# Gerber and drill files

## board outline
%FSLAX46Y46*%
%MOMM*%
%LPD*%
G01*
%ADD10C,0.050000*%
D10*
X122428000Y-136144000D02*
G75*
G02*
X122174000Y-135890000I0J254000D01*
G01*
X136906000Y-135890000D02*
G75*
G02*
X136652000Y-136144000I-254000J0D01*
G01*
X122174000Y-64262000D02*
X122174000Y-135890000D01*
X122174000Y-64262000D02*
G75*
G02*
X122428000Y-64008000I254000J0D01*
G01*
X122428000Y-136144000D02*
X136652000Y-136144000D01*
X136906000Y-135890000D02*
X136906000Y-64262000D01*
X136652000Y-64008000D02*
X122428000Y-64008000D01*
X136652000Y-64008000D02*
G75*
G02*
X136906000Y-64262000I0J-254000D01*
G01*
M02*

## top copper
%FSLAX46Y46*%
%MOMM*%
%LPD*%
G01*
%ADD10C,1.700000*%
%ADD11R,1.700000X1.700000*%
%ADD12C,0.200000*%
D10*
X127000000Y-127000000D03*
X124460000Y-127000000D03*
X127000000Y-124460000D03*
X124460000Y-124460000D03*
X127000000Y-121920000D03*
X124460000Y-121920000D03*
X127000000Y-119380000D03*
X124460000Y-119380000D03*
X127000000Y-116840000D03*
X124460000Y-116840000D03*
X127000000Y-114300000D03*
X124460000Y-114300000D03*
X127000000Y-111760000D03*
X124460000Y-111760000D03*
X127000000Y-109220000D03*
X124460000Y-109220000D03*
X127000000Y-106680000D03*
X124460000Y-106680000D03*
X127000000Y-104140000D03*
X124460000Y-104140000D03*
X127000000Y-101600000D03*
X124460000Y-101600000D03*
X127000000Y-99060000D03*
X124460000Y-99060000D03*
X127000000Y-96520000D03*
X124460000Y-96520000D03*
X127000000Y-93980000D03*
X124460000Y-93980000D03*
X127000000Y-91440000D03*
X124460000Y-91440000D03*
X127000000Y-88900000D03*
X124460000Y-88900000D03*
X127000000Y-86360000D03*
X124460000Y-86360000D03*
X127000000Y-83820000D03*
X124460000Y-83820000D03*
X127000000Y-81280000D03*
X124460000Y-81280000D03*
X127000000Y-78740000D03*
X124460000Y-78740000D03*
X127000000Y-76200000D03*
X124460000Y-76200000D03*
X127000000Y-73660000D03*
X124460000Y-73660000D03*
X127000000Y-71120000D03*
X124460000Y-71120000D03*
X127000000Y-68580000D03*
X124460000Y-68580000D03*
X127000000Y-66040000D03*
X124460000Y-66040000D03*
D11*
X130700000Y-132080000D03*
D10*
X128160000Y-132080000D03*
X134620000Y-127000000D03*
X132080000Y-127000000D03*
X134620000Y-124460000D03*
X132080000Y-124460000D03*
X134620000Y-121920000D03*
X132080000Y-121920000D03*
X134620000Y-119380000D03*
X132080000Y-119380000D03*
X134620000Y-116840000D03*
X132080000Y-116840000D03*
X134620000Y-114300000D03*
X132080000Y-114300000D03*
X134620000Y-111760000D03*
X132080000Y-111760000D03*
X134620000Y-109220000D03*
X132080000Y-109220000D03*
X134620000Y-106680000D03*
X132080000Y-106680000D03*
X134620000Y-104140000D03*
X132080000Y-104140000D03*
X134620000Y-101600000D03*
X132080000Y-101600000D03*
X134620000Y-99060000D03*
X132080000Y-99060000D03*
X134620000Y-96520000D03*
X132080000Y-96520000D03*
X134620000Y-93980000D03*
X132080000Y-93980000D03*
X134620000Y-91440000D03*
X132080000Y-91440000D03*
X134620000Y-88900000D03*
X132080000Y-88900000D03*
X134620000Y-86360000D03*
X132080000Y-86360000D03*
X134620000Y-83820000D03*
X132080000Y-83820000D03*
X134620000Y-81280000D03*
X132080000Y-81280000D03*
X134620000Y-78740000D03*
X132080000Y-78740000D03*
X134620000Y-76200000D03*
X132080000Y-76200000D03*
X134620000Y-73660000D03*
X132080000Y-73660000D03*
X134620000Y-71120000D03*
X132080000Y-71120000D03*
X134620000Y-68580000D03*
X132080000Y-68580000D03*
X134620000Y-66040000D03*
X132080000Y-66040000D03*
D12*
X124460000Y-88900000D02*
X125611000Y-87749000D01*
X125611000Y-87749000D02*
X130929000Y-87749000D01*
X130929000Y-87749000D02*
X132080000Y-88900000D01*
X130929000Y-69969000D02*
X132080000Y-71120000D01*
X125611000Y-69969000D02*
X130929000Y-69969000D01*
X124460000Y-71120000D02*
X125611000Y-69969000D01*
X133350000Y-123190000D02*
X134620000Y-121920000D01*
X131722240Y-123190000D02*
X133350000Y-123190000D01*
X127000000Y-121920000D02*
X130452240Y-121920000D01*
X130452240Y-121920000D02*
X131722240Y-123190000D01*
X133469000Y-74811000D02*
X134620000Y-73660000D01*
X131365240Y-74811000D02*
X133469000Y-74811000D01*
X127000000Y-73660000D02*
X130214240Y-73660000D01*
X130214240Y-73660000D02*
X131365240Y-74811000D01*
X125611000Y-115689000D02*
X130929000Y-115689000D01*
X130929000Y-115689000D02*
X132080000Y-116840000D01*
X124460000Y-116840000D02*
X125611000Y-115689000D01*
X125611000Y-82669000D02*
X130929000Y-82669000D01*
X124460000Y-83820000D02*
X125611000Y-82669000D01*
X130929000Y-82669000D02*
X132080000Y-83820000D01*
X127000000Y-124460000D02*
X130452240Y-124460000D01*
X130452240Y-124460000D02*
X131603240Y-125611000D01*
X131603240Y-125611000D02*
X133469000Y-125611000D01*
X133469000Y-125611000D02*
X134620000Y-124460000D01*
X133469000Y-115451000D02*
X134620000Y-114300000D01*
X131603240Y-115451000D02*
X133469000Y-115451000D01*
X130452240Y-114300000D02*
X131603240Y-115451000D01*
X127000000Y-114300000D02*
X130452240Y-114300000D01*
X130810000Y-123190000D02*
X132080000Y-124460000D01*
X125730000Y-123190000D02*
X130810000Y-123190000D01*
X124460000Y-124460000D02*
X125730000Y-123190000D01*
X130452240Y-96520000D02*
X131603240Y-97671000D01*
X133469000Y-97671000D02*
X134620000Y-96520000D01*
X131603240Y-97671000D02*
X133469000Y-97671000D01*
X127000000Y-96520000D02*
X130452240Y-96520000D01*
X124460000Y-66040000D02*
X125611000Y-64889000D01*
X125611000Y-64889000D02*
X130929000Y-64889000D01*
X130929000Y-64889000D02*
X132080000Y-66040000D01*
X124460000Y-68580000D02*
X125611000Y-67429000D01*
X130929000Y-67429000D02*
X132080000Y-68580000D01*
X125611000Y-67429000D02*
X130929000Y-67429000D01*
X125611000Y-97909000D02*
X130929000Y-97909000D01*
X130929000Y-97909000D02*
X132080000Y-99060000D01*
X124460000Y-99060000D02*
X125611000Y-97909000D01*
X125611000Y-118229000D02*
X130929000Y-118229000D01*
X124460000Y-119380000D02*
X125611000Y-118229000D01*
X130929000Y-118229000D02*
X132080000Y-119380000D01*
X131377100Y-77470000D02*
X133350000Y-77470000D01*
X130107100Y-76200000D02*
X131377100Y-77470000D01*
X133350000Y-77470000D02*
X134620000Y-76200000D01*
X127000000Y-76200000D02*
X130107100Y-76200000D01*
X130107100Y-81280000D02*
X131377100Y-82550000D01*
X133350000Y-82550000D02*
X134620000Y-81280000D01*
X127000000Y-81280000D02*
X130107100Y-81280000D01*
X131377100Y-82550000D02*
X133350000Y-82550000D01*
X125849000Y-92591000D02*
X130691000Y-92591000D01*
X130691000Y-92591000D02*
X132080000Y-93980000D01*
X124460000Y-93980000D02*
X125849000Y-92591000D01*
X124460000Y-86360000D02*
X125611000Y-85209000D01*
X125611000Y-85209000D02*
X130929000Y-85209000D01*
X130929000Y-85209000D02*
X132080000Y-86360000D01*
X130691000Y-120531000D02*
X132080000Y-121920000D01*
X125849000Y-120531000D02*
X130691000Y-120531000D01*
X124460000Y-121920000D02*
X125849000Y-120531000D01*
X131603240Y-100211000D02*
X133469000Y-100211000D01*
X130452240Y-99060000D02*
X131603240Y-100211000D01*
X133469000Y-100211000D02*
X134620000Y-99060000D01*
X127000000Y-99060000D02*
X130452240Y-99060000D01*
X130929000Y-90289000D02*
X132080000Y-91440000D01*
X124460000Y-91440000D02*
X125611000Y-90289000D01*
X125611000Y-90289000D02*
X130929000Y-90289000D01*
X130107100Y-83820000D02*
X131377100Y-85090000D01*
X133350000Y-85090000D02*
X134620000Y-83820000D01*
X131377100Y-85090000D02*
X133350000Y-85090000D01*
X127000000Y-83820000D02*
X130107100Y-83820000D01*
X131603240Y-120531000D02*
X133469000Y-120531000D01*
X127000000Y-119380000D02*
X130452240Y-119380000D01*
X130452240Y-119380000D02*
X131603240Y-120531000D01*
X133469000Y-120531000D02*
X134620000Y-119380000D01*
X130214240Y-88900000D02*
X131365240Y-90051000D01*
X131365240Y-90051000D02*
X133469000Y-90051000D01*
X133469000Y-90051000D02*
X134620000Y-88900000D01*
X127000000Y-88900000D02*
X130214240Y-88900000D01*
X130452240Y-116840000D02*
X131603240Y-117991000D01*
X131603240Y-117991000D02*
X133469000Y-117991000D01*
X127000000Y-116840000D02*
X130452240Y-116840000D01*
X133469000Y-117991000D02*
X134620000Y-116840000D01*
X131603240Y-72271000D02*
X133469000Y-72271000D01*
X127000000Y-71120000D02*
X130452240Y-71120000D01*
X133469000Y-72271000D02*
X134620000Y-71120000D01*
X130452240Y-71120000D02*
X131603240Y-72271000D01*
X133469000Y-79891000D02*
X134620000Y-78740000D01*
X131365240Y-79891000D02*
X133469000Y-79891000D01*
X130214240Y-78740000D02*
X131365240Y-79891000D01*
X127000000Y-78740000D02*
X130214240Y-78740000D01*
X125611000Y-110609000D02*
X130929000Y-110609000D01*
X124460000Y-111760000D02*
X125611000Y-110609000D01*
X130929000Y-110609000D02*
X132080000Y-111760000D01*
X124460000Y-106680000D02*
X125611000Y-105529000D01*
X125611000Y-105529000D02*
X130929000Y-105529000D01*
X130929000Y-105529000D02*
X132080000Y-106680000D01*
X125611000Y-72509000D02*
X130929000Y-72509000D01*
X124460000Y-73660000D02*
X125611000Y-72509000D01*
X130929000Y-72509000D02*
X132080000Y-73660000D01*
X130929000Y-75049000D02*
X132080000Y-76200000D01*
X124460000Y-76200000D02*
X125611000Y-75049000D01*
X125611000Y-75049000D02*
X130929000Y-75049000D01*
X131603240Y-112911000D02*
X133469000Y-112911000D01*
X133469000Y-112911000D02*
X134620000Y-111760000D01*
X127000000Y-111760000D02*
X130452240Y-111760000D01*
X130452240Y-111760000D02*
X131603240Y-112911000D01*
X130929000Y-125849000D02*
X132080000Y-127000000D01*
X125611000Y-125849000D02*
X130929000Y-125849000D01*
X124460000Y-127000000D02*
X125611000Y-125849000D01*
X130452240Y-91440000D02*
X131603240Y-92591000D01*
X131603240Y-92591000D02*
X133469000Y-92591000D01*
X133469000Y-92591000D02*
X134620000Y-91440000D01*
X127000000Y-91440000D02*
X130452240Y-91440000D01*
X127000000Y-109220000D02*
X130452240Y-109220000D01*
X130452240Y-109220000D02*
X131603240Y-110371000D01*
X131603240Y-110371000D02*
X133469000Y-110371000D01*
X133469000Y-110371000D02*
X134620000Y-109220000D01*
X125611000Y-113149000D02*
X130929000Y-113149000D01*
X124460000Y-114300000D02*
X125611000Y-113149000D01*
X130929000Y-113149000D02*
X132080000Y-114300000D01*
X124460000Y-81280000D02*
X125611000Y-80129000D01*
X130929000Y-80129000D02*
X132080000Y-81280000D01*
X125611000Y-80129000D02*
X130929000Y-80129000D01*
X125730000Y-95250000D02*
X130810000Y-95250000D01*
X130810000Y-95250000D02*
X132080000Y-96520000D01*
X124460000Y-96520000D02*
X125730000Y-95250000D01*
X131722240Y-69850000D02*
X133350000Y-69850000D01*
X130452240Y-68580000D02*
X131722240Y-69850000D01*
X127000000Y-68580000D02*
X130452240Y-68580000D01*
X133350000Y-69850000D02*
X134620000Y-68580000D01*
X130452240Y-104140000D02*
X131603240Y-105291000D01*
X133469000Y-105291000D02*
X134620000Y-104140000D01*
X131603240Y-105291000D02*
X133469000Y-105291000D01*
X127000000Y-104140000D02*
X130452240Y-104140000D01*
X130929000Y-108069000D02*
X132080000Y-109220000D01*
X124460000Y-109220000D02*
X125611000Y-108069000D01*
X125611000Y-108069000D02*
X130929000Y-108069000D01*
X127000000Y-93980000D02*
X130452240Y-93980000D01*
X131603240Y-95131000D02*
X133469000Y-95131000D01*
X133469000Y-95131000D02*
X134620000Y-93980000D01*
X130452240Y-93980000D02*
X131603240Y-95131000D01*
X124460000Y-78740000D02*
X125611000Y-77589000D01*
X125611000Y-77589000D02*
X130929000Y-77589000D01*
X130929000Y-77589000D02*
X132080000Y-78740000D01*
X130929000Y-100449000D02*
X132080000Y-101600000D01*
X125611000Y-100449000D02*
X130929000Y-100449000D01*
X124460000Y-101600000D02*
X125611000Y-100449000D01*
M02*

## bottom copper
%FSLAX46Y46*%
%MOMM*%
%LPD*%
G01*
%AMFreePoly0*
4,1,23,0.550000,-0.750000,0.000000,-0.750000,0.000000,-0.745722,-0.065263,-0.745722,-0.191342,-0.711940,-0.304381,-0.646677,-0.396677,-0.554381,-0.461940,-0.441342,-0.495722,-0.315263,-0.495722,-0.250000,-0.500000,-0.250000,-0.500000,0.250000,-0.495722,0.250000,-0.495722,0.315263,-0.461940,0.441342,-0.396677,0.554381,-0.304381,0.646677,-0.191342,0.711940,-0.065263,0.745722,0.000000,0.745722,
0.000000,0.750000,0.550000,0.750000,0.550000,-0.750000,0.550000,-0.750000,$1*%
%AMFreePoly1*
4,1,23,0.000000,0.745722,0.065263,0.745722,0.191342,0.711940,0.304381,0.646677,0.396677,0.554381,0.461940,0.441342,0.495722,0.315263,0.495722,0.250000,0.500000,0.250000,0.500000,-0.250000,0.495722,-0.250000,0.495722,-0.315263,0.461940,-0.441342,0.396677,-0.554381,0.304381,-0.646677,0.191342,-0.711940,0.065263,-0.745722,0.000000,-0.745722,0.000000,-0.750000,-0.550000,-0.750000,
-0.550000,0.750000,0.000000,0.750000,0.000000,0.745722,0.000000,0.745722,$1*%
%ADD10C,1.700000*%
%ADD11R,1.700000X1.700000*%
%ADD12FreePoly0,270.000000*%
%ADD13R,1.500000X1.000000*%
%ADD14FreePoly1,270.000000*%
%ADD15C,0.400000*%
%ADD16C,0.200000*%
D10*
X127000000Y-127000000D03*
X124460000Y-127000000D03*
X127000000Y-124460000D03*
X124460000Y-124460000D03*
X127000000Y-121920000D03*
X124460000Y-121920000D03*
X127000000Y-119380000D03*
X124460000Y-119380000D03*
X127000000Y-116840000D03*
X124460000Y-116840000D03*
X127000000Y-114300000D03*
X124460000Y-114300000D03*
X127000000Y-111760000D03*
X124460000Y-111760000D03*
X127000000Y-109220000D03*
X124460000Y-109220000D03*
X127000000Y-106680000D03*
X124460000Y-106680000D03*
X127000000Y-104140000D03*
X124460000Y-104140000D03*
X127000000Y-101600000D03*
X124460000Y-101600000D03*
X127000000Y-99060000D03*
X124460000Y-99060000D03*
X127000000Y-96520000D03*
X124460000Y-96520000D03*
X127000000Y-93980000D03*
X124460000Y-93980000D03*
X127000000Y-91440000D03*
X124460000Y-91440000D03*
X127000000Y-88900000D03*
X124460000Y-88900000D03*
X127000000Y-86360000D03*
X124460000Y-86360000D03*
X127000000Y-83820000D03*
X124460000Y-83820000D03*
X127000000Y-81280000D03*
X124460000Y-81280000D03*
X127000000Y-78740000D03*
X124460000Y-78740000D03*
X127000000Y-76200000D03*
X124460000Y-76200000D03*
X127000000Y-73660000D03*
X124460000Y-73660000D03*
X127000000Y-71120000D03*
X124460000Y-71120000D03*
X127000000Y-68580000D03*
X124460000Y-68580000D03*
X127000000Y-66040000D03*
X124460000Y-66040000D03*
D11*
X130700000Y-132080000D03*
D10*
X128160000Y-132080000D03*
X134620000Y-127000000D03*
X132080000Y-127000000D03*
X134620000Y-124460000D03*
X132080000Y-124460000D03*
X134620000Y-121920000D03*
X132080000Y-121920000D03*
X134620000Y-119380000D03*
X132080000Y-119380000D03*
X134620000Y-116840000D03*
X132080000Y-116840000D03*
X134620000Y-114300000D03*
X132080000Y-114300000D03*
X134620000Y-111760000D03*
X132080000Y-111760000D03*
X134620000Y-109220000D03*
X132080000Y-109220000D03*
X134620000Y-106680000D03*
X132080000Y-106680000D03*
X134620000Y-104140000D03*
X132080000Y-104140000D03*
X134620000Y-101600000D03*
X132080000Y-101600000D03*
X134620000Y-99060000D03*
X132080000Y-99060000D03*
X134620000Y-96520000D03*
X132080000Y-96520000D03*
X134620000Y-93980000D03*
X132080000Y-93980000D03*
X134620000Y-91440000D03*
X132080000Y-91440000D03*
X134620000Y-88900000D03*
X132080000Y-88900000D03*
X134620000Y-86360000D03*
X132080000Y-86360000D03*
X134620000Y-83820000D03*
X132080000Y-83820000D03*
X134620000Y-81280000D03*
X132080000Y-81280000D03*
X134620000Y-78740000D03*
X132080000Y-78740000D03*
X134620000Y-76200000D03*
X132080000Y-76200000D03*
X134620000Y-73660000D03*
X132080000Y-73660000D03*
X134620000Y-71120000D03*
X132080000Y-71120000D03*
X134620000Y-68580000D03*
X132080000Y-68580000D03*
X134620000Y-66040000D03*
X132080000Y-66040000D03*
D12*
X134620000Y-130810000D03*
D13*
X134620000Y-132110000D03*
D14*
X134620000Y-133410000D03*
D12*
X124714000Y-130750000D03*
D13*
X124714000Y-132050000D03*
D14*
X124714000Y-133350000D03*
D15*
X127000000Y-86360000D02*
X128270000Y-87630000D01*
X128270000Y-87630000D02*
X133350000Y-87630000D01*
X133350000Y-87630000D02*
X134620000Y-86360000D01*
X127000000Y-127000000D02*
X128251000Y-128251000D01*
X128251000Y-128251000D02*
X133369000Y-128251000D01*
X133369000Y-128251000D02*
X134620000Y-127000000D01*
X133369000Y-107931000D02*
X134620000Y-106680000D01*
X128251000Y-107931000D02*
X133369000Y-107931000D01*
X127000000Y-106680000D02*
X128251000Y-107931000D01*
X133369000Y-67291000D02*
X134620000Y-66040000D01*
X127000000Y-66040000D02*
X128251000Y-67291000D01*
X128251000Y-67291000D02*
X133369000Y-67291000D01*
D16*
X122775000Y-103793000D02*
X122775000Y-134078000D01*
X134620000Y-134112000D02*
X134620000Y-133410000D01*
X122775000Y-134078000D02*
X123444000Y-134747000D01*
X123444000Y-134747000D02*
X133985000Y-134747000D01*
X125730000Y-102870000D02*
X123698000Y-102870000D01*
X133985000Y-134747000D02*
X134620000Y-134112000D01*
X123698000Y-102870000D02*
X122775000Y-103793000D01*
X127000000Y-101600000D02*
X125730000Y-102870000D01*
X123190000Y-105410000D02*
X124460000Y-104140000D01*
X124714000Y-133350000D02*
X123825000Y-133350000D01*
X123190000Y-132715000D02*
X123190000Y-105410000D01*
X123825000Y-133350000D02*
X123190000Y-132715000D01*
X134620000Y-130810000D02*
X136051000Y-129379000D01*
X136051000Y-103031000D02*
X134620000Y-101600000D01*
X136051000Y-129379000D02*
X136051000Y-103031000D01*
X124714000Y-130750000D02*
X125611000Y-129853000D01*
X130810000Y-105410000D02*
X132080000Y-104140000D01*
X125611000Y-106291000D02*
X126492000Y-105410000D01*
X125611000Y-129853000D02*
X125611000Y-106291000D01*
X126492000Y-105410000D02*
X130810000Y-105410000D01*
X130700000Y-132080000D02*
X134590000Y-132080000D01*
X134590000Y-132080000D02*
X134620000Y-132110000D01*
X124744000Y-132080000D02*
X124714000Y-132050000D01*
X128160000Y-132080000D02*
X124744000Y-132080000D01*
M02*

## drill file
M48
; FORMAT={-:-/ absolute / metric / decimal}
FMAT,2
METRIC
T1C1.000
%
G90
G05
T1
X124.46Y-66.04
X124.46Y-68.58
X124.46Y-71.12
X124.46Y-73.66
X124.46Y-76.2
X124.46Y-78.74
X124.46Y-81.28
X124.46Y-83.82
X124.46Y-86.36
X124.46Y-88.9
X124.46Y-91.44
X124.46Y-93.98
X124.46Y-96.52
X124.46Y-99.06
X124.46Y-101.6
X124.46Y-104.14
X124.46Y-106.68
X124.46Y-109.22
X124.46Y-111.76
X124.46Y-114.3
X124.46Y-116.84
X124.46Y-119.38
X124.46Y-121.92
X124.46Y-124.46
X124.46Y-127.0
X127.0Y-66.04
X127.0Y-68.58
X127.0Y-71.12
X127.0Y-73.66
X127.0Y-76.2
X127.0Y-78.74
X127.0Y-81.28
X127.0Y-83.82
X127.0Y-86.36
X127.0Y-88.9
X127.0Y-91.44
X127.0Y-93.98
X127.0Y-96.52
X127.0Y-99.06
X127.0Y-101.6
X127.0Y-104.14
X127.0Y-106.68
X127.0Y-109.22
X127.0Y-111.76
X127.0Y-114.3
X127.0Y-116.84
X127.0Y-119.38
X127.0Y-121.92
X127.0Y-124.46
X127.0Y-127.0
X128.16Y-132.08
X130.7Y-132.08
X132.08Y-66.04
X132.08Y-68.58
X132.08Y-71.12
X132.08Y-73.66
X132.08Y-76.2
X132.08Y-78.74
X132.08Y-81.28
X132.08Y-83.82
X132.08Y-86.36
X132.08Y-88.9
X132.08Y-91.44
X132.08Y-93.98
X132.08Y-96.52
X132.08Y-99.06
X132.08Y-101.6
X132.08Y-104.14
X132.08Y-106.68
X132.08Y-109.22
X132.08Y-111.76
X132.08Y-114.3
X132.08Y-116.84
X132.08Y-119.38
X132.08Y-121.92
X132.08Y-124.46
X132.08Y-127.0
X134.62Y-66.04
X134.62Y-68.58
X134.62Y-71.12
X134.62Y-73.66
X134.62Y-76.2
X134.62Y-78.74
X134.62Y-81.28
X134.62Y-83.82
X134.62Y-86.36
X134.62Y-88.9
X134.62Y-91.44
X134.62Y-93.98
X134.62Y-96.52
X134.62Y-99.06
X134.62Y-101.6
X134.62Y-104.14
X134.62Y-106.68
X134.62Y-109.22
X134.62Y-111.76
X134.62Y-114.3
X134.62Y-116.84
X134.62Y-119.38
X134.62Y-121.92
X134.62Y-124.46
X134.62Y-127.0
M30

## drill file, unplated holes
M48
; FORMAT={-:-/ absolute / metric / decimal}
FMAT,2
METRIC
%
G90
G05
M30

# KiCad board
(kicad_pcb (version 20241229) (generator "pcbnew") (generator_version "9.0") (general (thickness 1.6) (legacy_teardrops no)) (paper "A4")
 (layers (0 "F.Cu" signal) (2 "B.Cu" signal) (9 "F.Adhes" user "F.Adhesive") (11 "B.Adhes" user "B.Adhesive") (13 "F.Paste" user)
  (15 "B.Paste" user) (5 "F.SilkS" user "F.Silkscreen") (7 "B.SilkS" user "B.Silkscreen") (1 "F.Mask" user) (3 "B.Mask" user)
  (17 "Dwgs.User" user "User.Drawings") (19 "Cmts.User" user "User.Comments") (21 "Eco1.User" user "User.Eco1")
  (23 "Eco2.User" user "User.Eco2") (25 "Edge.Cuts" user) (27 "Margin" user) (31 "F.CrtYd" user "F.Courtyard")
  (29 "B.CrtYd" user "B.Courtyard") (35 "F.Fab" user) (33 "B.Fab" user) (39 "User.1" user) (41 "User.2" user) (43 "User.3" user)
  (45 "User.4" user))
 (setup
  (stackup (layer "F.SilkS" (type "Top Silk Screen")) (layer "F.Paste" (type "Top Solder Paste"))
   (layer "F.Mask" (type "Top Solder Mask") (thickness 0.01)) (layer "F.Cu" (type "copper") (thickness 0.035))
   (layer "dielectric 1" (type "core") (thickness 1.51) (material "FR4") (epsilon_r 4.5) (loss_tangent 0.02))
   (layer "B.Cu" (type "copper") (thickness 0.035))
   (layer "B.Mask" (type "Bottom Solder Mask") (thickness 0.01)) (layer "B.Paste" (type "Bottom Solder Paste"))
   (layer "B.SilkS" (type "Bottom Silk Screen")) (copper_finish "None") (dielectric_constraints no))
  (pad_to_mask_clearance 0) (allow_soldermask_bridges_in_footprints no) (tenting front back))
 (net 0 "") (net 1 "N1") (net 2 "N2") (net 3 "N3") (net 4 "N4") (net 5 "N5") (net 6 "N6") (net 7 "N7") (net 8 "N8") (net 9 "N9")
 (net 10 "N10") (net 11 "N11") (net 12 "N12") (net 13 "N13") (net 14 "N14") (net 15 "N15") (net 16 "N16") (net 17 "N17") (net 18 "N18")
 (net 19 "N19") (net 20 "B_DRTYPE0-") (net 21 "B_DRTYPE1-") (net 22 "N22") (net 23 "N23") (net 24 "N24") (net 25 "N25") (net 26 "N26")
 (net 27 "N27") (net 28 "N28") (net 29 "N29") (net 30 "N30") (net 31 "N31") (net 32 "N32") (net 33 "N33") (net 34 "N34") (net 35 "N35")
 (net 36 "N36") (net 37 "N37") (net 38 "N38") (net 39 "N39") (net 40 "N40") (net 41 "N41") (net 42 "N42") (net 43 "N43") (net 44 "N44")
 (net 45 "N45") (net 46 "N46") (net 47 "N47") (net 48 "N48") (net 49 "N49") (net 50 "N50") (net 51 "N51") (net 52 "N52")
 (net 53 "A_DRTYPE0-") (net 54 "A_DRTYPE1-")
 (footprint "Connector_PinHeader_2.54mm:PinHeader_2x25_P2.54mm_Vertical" (layer "F.Cu") (at 127 127 180)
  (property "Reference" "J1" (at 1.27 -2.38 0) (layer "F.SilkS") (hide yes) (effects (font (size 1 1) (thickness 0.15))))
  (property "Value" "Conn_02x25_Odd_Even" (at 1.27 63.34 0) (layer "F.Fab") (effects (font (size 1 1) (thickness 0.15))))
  (pad "1" thru_hole circle (at 0 0 180) (size 1.7 1.7) (drill 1) (layers "*.Cu" "*.Mask") (remove_unused_layers no) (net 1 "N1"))
  (pad "2" thru_hole circle (at 2.54 0 180) (size 1.7 1.7) (drill 1) (layers "*.Cu" "*.Mask") (remove_unused_layers no) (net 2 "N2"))
  (pad "3" thru_hole circle (at 0 2.54 180) (size 1.7 1.7) (drill 1) (layers "*.Cu" "*.Mask") (remove_unused_layers no) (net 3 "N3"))
  (pad "4" thru_hole circle (at 2.54 2.54 180) (size 1.7 1.7) (drill 1) (layers "*.Cu" "*.Mask") (remove_unused_layers no) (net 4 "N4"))
  (pad "5" thru_hole circle (at 0 5.08 180) (size 1.7 1.7) (drill 1) (layers "*.Cu" "*.Mask") (remove_unused_layers no) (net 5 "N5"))
  (pad "6" thru_hole circle (at 2.54 5.08 180) (size 1.7 1.7) (drill 1) (layers "*.Cu" "*.Mask") (remove_unused_layers no) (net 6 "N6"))
  (pad "7" thru_hole circle (at 0 7.62 180) (size 1.7 1.7) (drill 1) (layers "*.Cu" "*.Mask") (remove_unused_layers no) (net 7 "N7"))
  (pad "8" thru_hole circle (at 2.54 7.62 180) (size 1.7 1.7) (drill 1) (layers "*.Cu" "*.Mask") (remove_unused_layers no) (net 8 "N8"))
  (pad "9" thru_hole circle (at 0 10.16 180) (size 1.7 1.7) (drill 1) (layers "*.Cu" "*.Mask") (remove_unused_layers no) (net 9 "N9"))
  (pad "10" thru_hole circle (at 2.54 10.16 180) (size 1.7 1.7) (drill 1) (layers "*.Cu" "*.Mask") (remove_unused_layers no) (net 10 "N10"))
  (pad "11" thru_hole circle (at 0 12.7 180) (size 1.7 1.7) (drill 1) (layers "*.Cu" "*.Mask") (remove_unused_layers no) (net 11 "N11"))
  (pad "12" thru_hole circle (at 2.54 12.7 180) (size 1.7 1.7) (drill 1) (layers "*.Cu" "*.Mask") (remove_unused_layers no) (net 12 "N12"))
  (pad "13" thru_hole circle (at 0 15.24 180) (size 1.7 1.7) (drill 1) (layers "*.Cu" "*.Mask") (remove_unused_layers no) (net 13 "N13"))
  (pad "14" thru_hole circle (at 2.54 15.24 180) (size 1.7 1.7) (drill 1) (layers "*.Cu" "*.Mask") (remove_unused_layers no) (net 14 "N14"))
  (pad "15" thru_hole circle (at 0 17.78 180) (size 1.7 1.7) (drill 1) (layers "*.Cu" "*.Mask") (remove_unused_layers no) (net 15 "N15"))
  (pad "16" thru_hole circle (at 2.54 17.78 180) (size 1.7 1.7) (drill 1) (layers "*.Cu" "*.Mask") (remove_unused_layers no) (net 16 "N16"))
  (pad "17" thru_hole circle (at 0 20.32 180) (size 1.7 1.7) (drill 1) (layers "*.Cu" "*.Mask") (remove_unused_layers no) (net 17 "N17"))
  (pad "18" thru_hole circle (at 2.54 20.32 180) (size 1.7 1.7) (drill 1) (layers "*.Cu" "*.Mask") (remove_unused_layers no) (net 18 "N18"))
  (pad "19" thru_hole circle (at 0 22.86 180) (size 1.7 1.7) (drill 1) (layers "*.Cu" "*.Mask") (remove_unused_layers no) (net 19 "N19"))
  (pad "20" thru_hole circle (at 2.54 22.86 180) (size 1.7 1.7) (drill 1) (layers "*.Cu" "*.Mask") (remove_unused_layers no)
   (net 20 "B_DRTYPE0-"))
  (pad "21" thru_hole circle (at 0 25.4 180) (size 1.7 1.7) (drill 1) (layers "*.Cu" "*.Mask") (remove_unused_layers no)
   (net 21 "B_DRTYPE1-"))
  (pad "22" thru_hole circle (at 2.54 25.4 180) (size 1.7 1.7) (drill 1) (layers "*.Cu" "*.Mask") (remove_unused_layers no) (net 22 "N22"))
  (pad "23" thru_hole circle (at 0 27.94 180) (size 1.7 1.7) (drill 1) (layers "*.Cu" "*.Mask") (remove_unused_layers no) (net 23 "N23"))
  (pad "24" thru_hole circle (at 2.54 27.94 180) (size 1.7 1.7) (drill 1) (layers "*.Cu" "*.Mask") (remove_unused_layers no) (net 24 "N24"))
  (pad "25" thru_hole circle (at 0 30.48 180) (size 1.7 1.7) (drill 1) (layers "*.Cu" "*.Mask") (remove_unused_layers no) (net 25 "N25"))
  (pad "26" thru_hole circle (at 2.54 30.48 180) (size 1.7 1.7) (drill 1) (layers "*.Cu" "*.Mask") (remove_unused_layers no) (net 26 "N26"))
  (pad "27" thru_hole circle (at 0 33.02 180) (size 1.7 1.7) (drill 1) (layers "*.Cu" "*.Mask") (remove_unused_layers no) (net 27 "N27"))
  (pad "28" thru_hole circle (at 2.54 33.02 180) (size 1.7 1.7) (drill 1) (layers "*.Cu" "*.Mask") (remove_unused_layers no) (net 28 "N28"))
  (pad "29" thru_hole circle (at 0 35.56 180) (size 1.7 1.7) (drill 1) (layers "*.Cu" "*.Mask") (remove_unused_layers no) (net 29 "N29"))
  (pad "30" thru_hole circle (at 2.54 35.56 180) (size 1.7 1.7) (drill 1) (layers "*.Cu" "*.Mask") (remove_unused_layers no) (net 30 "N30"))
  (pad "31" thru_hole circle (at 0 38.1 180) (size 1.7 1.7) (drill 1) (layers "*.Cu" "*.Mask") (remove_unused_layers no) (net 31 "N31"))
  (pad "32" thru_hole circle (at 2.54 38.1 180) (size 1.7 1.7) (drill 1) (layers "*.Cu" "*.Mask") (remove_unused_layers no) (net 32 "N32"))
  (pad "33" thru_hole circle (at 0 40.64 180) (size 1.7 1.7) (drill 1) (layers "*.Cu" "*.Mask") (remove_unused_layers no) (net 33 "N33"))
  (pad "34" thru_hole circle (at 2.54 40.64 180) (size 1.7 1.7) (drill 1) (layers "*.Cu" "*.Mask") (remove_unused_layers no) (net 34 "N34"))
  (pad "35" thru_hole circle (at 0 43.18 180) (size 1.7 1.7) (drill 1) (layers "*.Cu" "*.Mask") (remove_unused_layers no) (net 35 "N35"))
  (pad "36" thru_hole circle (at 2.54 43.18 180) (size 1.7 1.7) (drill 1) (layers "*.Cu" "*.Mask") (remove_unused_layers no) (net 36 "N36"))
  (pad "37" thru_hole circle (at 0 45.72 180) (size 1.7 1.7) (drill 1) (layers "*.Cu" "*.Mask") (remove_unused_layers no) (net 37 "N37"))
  (pad "38" thru_hole circle (at 2.54 45.72 180) (size 1.7 1.7) (drill 1) (layers "*.Cu" "*.Mask") (remove_unused_layers no) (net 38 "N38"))
  (pad "39" thru_hole circle (at 0 48.26 180) (size 1.7 1.7) (drill 1) (layers "*.Cu" "*.Mask") (remove_unused_layers no) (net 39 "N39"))
  (pad "40" thru_hole circle (at 2.54 48.26 180) (size 1.7 1.7) (drill 1) (layers "*.Cu" "*.Mask") (remove_unused_layers no) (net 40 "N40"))
  (pad "41" thru_hole circle (at 0 50.8 180) (size 1.7 1.7) (drill 1) (layers "*.Cu" "*.Mask") (remove_unused_layers no) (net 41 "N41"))
  (pad "42" thru_hole circle (at 2.54 50.8 180) (size 1.7 1.7) (drill 1) (layers "*.Cu" "*.Mask") (remove_unused_layers no) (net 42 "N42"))
  (pad "43" thru_hole circle (at 0 53.34 180) (size 1.7 1.7) (drill 1) (layers "*.Cu" "*.Mask") (remove_unused_layers no) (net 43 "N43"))
  (pad "44" thru_hole circle (at 2.54 53.34 180) (size 1.7 1.7) (drill 1) (layers "*.Cu" "*.Mask") (remove_unused_layers no) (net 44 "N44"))
  (pad "45" thru_hole circle (at 0 55.88 180) (size 1.7 1.7) (drill 1) (layers "*.Cu" "*.Mask") (remove_unused_layers no) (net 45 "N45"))
  (pad "46" thru_hole circle (at 2.54 55.88 180) (size 1.7 1.7) (drill 1) (layers "*.Cu" "*.Mask") (remove_unused_layers no) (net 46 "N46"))
  (pad "47" thru_hole circle (at 0 58.42 180) (size 1.7 1.7) (drill 1) (layers "*.Cu" "*.Mask") (remove_unused_layers no) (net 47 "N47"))
  (pad "48" thru_hole circle (at 2.54 58.42 180) (size 1.7 1.7) (drill 1) (layers "*.Cu" "*.Mask") (remove_unused_layers no) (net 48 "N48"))
  (pad "49" thru_hole circle (at 0 60.96 180) (size 1.7 1.7) (drill 1) (layers "*.Cu" "*.Mask") (remove_unused_layers no) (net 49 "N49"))
  (pad "50" thru_hole circle (at 2.54 60.96 180) (size 1.7 1.7) (drill 1) (layers "*.Cu" "*.Mask") (remove_unused_layers no) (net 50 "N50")))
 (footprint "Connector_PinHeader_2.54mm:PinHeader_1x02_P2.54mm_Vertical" (layer "F.Cu") (at 130.7 132.08 -90)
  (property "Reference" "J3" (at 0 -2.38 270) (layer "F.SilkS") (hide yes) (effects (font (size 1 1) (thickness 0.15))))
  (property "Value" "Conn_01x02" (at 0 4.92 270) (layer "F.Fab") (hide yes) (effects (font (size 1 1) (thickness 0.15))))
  (pad "1" thru_hole rect (at 0 0 270) (size 1.7 1.7) (drill 1) (layers "*.Cu" "*.Mask") (remove_unused_layers no) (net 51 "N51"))
  (pad "2" thru_hole circle (at 0 2.54 270) (size 1.7 1.7) (drill 1) (layers "*.Cu" "*.Mask") (remove_unused_layers no) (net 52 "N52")))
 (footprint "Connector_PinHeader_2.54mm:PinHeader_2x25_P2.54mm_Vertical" (layer "F.Cu") (at 134.62 127 180)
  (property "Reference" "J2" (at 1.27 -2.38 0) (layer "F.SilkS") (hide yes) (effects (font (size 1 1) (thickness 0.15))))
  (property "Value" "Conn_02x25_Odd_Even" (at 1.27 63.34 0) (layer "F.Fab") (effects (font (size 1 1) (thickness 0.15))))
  (pad "1" thru_hole circle (at 0 0 180) (size 1.7 1.7) (drill 1) (layers "*.Cu" "*.Mask") (remove_unused_layers no) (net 1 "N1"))
  (pad "2" thru_hole circle (at 2.54 0 180) (size 1.7 1.7) (drill 1) (layers "*.Cu" "*.Mask") (remove_unused_layers no) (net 2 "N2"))
  (pad "3" thru_hole circle (at 0 2.54 180) (size 1.7 1.7) (drill 1) (layers "*.Cu" "*.Mask") (remove_unused_layers no) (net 3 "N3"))
  (pad "4" thru_hole circle (at 2.54 2.54 180) (size 1.7 1.7) (drill 1) (layers "*.Cu" "*.Mask") (remove_unused_layers no) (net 4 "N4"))
  (pad "5" thru_hole circle (at 0 5.08 180) (size 1.7 1.7) (drill 1) (layers "*.Cu" "*.Mask") (remove_unused_layers no) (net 5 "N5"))
  (pad "6" thru_hole circle (at 2.54 5.08 180) (size 1.7 1.7) (drill 1) (layers "*.Cu" "*.Mask") (remove_unused_layers no) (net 6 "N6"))
  (pad "7" thru_hole circle (at 0 7.62 180) (size 1.7 1.7) (drill 1) (layers "*.Cu" "*.Mask") (remove_unused_layers no) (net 7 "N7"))
  (pad "8" thru_hole circle (at 2.54 7.62 180) (size 1.7 1.7) (drill 1) (layers "*.Cu" "*.Mask") (remove_unused_layers no) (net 8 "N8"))
  (pad "9" thru_hole circle (at 0 10.16 180) (size 1.7 1.7) (drill 1) (layers "*.Cu" "*.Mask") (remove_unused_layers no) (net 9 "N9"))
  (pad "10" thru_hole circle (at 2.54 10.16 180) (size 1.7 1.7) (drill 1) (layers "*.Cu" "*.Mask") (remove_unused_layers no) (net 10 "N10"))
  (pad "11" thru_hole circle (at 0 12.7 180) (size 1.7 1.7) (drill 1) (layers "*.Cu" "*.Mask") (remove_unused_layers no) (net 11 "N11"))
  (pad "12" thru_hole circle (at 2.54 12.7 180) (size 1.7 1.7) (drill 1) (layers "*.Cu" "*.Mask") (remove_unused_layers no) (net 12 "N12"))
  (pad "13" thru_hole circle (at 0 15.24 180) (size 1.7 1.7) (drill 1) (layers "*.Cu" "*.Mask") (remove_unused_layers no) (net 13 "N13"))
  (pad "14" thru_hole circle (at 2.54 15.24 180) (size 1.7 1.7) (drill 1) (layers "*.Cu" "*.Mask") (remove_unused_layers no) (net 14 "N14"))
  (pad "15" thru_hole circle (at 0 17.78 180) (size 1.7 1.7) (drill 1) (layers "*.Cu" "*.Mask") (remove_unused_layers no) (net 15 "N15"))
  (pad "16" thru_hole circle (at 2.54 17.78 180) (size 1.7 1.7) (drill 1) (layers "*.Cu" "*.Mask") (remove_unused_layers no) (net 16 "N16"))
  (pad "17" thru_hole circle (at 0 20.32 180) (size 1.7 1.7) (drill 1) (layers "*.Cu" "*.Mask") (remove_unused_layers no) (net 17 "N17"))
  (pad "18" thru_hole circle (at 2.54 20.32 180) (size 1.7 1.7) (drill 1) (layers "*.Cu" "*.Mask") (remove_unused_layers no) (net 18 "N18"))
  (pad "19" thru_hole circle (at 0 22.86 180) (size 1.7 1.7) (drill 1) (layers "*.Cu" "*.Mask") (remove_unused_layers no) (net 19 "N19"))
  (pad "20" thru_hole circle (at 2.54 22.86 180) (size 1.7 1.7) (drill 1) (layers "*.Cu" "*.Mask") (remove_unused_layers no)
   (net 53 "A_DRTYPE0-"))
  (pad "21" thru_hole circle (at 0 25.4 180) (size 1.7 1.7) (drill 1) (layers "*.Cu" "*.Mask") (remove_unused_layers no)
   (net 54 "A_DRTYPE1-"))
  (pad "22" thru_hole circle (at 2.54 25.4 180) (size 1.7 1.7) (drill 1) (layers "*.Cu" "*.Mask") (remove_unused_layers no) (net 22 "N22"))
  (pad "23" thru_hole circle (at 0 27.94 180) (size 1.7 1.7) (drill 1) (layers "*.Cu" "*.Mask") (remove_unused_layers no) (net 23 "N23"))
  (pad "24" thru_hole circle (at 2.54 27.94 180) (size 1.7 1.7) (drill 1) (layers "*.Cu" "*.Mask") (remove_unused_layers no) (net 24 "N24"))
  (pad "25" thru_hole circle (at 0 30.48 180) (size 1.7 1.7) (drill 1) (layers "*.Cu" "*.Mask") (remove_unused_layers no) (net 25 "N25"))
  (pad "26" thru_hole circle (at 2.54 30.48 180) (size 1.7 1.7) (drill 1) (layers "*.Cu" "*.Mask") (remove_unused_layers no) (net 26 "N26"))
  (pad "27" thru_hole circle (at 0 33.02 180) (size 1.7 1.7) (drill 1) (layers "*.Cu" "*.Mask") (remove_unused_layers no) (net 27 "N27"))
  (pad "28" thru_hole circle (at 2.54 33.02 180) (size 1.7 1.7) (drill 1) (layers "*.Cu" "*.Mask") (remove_unused_layers no) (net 28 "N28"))
  (pad "29" thru_hole circle (at 0 35.56 180) (size 1.7 1.7) (drill 1) (layers "*.Cu" "*.Mask") (remove_unused_layers no) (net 29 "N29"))
  (pad "30" thru_hole circle (at 2.54 35.56 180) (size 1.7 1.7) (drill 1) (layers "*.Cu" "*.Mask") (remove_unused_layers no) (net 30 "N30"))
  (pad "31" thru_hole circle (at 0 38.1 180) (size 1.7 1.7) (drill 1) (layers "*.Cu" "*.Mask") (remove_unused_layers no) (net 31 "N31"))
  (pad "32" thru_hole circle (at 2.54 38.1 180) (size 1.7 1.7) (drill 1) (layers "*.Cu" "*.Mask") (remove_unused_layers no) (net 32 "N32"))
  (pad "33" thru_hole circle (at 0 40.64 180) (size 1.7 1.7) (drill 1) (layers "*.Cu" "*.Mask") (remove_unused_layers no) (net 33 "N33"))
  (pad "34" thru_hole circle (at 2.54 40.64 180) (size 1.7 1.7) (drill 1) (layers "*.Cu" "*.Mask") (remove_unused_layers no) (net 34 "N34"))
  (pad "35" thru_hole circle (at 0 43.18 180) (size 1.7 1.7) (drill 1) (layers "*.Cu" "*.Mask") (remove_unused_layers no) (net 35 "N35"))
  (pad "36" thru_hole circle (at 2.54 43.18 180) (size 1.7 1.7) (drill 1) (layers "*.Cu" "*.Mask") (remove_unused_layers no) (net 36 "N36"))
  (pad "37" thru_hole circle (at 0 45.72 180) (size 1.7 1.7) (drill 1) (layers "*.Cu" "*.Mask") (remove_unused_layers no) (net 37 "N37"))
  (pad "38" thru_hole circle (at 2.54 45.72 180) (size 1.7 1.7) (drill 1) (layers "*.Cu" "*.Mask") (remove_unused_layers no) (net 38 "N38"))
  (pad "39" thru_hole circle (at 0 48.26 180) (size 1.7 1.7) (drill 1) (layers "*.Cu" "*.Mask") (remove_unused_layers no) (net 39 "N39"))
  (pad "40" thru_hole circle (at 2.54 48.26 180) (size 1.7 1.7) (drill 1) (layers "*.Cu" "*.Mask") (remove_unused_layers no) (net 40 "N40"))
  (pad "41" thru_hole circle (at 0 50.8 180) (size 1.7 1.7) (drill 1) (layers "*.Cu" "*.Mask") (remove_unused_layers no) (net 41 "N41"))
  (pad "42" thru_hole circle (at 2.54 50.8 180) (size 1.7 1.7) (drill 1) (layers "*.Cu" "*.Mask") (remove_unused_layers no) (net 42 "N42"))
  (pad "43" thru_hole circle (at 0 53.34 180) (size 1.7 1.7) (drill 1) (layers "*.Cu" "*.Mask") (remove_unused_layers no) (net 43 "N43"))
  (pad "44" thru_hole circle (at 2.54 53.34 180) (size 1.7 1.7) (drill 1) (layers "*.Cu" "*.Mask") (remove_unused_layers no) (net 44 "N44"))
  (pad "45" thru_hole circle (at 0 55.88 180) (size 1.7 1.7) (drill 1) (layers "*.Cu" "*.Mask") (remove_unused_layers no) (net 45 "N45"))
  (pad "46" thru_hole circle (at 2.54 55.88 180) (size 1.7 1.7) (drill 1) (layers "*.Cu" "*.Mask") (remove_unused_layers no) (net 46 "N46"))
  (pad "47" thru_hole circle (at 0 58.42 180) (size 1.7 1.7) (drill 1) (layers "*.Cu" "*.Mask") (remove_unused_layers no) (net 47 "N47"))
  (pad "48" thru_hole circle (at 2.54 58.42 180) (size 1.7 1.7) (drill 1) (layers "*.Cu" "*.Mask") (remove_unused_layers no) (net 48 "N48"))
  (pad "49" thru_hole circle (at 0 60.96 180) (size 1.7 1.7) (drill 1) (layers "*.Cu" "*.Mask") (remove_unused_layers no) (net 49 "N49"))
  (pad "50" thru_hole circle (at 2.54 60.96 180) (size 1.7 1.7) (drill 1) (layers "*.Cu" "*.Mask") (remove_unused_layers no) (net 50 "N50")))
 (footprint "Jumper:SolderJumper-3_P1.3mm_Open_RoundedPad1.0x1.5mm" (layer "B.Cu") (at 134.62 132.11 -90)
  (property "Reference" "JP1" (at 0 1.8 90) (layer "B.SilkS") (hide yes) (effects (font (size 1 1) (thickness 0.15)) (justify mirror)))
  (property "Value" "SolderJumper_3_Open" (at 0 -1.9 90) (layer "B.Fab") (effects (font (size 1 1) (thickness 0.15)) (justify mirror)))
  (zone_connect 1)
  (pad "1" smd custom (at -1.3 0 270) (size 1 0.5) (layers "B.Cu" "B.Mask") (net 54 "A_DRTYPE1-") (zone_connect 2) (thermal_bridge_angle 45)
   (options (clearance outline) (anchor rect)) (primitives))
  (pad "2" smd rect (at 0 0 270) (size 1 1.5) (layers "B.Cu" "B.Mask") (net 51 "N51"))
  (pad "3" smd custom (at 1.3 0 270) (size 1 0.5) (layers "B.Cu" "B.Mask") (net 21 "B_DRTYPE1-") (zone_connect 2) (thermal_bridge_angle 45)
   (options (clearance outline) (anchor rect)) (primitives)))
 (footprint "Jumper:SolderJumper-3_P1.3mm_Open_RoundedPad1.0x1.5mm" (layer "B.Cu") (at 124.714 132.05 -90)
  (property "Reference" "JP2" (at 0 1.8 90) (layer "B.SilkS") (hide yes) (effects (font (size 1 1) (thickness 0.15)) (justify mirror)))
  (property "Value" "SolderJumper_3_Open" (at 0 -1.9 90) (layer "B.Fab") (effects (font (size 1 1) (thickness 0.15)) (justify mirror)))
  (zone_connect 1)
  (pad "1" smd custom (at -1.3 0 270) (size 1 0.5) (layers "B.Cu" "B.Mask") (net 53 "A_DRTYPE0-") (zone_connect 2) (thermal_bridge_angle 45)
   (options (clearance outline) (anchor rect)) (primitives))
  (pad "2" smd rect (at 0 0 270) (size 1 1.5) (layers "B.Cu" "B.Mask") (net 52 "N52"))
  (pad "3" smd custom (at 1.3 0 270) (size 1 0.5) (layers "B.Cu" "B.Mask") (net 20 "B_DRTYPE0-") (zone_connect 2) (thermal_bridge_angle 45)
   (options (clearance outline) (anchor rect)) (primitives)))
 (gr_arc (start 122.428 136.144) (mid 122.248395 136.069605) (end 122.174 135.89) (stroke (width 0.05) (type default)) (layer "Edge.Cuts"))
 (gr_arc (start 136.906 135.89) (mid 136.831605 136.069605) (end 136.652 136.144) (stroke (width 0.05) (type default)) (layer "Edge.Cuts"))
 (gr_line (start 122.174 64.262) (end 122.174 135.89) (stroke (width 0.05) (type default)) (layer "Edge.Cuts"))
 (gr_arc (start 122.174 64.262) (mid 122.248395 64.082395) (end 122.428 64.008) (stroke (width 0.05) (type default)) (layer "Edge.Cuts"))
 (gr_line (start 122.428 136.144) (end 136.652 136.144) (stroke (width 0.05) (type default)) (layer "Edge.Cuts"))
 (gr_line (start 136.906 135.89) (end 136.906 64.262) (stroke (width 0.05) (type default)) (layer "Edge.Cuts"))
 (gr_line (start 136.652 64.008) (end 122.428 64.008) (stroke (width 0.05) (type default)) (layer "Edge.Cuts"))
 (gr_arc (start 136.652 64.008) (mid 136.831605 64.082395) (end 136.906 64.262) (stroke (width 0.05) (type default)) (layer "Edge.Cuts"))
 (segment (start 124.46 88.9) (end 125.611 87.749) (width 0.2) (layer "F.Cu") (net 32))
 (segment (start 125.611 87.749) (end 130.929 87.749) (width 0.2) (layer "F.Cu") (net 32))
 (segment (start 130.929 87.749) (end 132.08 88.9) (width 0.2) (layer "F.Cu") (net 32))
 (segment (start 130.929 69.969) (end 132.08 71.12) (width 0.2) (layer "F.Cu") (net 46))
 (segment (start 125.611 69.969) (end 130.929 69.969) (width 0.2) (layer "F.Cu") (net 46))
 (segment (start 124.46 71.12) (end 125.611 69.969) (width 0.2) (layer "F.Cu") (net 46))
 (segment (start 133.35 123.19) (end 134.62 121.92) (width 0.2) (layer "F.Cu") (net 5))
 (segment (start 131.72224 123.19) (end 133.35 123.19) (width 0.2) (layer "F.Cu") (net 5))
 (segment (start 127 121.92) (end 130.45224 121.92) (width 0.2) (layer "F.Cu") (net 5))
 (segment (start 130.45224 121.92) (end 131.72224 123.19) (width 0.2) (layer "F.Cu") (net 5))
 (segment (start 133.469 74.811) (end 134.62 73.66) (width 0.2) (layer "F.Cu") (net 43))
 (segment (start 131.36524 74.811) (end 133.469 74.811) (width 0.2) (layer "F.Cu") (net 43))
 (segment (start 127 73.66) (end 130.21424 73.66) (width 0.2) (layer "F.Cu") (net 43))
 (segment (start 130.21424 73.66) (end 131.36524 74.811) (width 0.2) (layer "F.Cu") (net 43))
 (segment (start 125.611 115.689) (end 130.929 115.689) (width 0.2) (layer "F.Cu") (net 10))
 (segment (start 130.929 115.689) (end 132.08 116.84) (width 0.2) (layer "F.Cu") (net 10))
 (segment (start 124.46 116.84) (end 125.611 115.689) (width 0.2) (layer "F.Cu") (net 10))
 (segment (start 125.611 82.669) (end 130.929 82.669) (width 0.2) (layer "F.Cu") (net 36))
 (segment (start 124.46 83.82) (end 125.611 82.669) (width 0.2) (layer "F.Cu") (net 36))
 (segment (start 130.929 82.669) (end 132.08 83.82) (width 0.2) (layer "F.Cu") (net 36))
 (segment (start 127 124.46) (end 130.45224 124.46) (width 0.2) (layer "F.Cu") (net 3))
 (segment (start 130.45224 124.46) (end 131.60324 125.611) (width 0.2) (layer "F.Cu") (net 3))
 (segment (start 131.60324 125.611) (end 133.469 125.611) (width 0.2) (layer "F.Cu") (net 3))
 (segment (start 133.469 125.611) (end 134.62 124.46) (width 0.2) (layer "F.Cu") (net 3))
 (segment (start 133.469 115.451) (end 134.62 114.3) (width 0.2) (layer "F.Cu") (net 11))
 (segment (start 131.60324 115.451) (end 133.469 115.451) (width 0.2) (layer "F.Cu") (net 11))
 (segment (start 130.45224 114.3) (end 131.60324 115.451) (width 0.2) (layer "F.Cu") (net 11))
 (segment (start 127 114.3) (end 130.45224 114.3) (width 0.2) (layer "F.Cu") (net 11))
 (segment (start 130.81 123.19) (end 132.08 124.46) (width 0.2) (layer "F.Cu") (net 4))
 (segment (start 125.73 123.19) (end 130.81 123.19) (width 0.2) (layer "F.Cu") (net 4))
 (segment (start 124.46 124.46) (end 125.73 123.19) (width 0.2) (layer "F.Cu") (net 4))
 (segment (start 130.45224 96.52) (end 131.60324 97.671) (width 0.2) (layer "F.Cu") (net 25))
 (segment (start 133.469 97.671) (end 134.62 96.52) (width 0.2) (layer "F.Cu") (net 25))
 (segment (start 131.60324 97.671) (end 133.469 97.671) (width 0.2) (layer "F.Cu") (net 25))
 (segment (start 127 96.52) (end 130.45224 96.52) (width 0.2) (layer "F.Cu") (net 25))
 (segment (start 127 86.36) (end 128.27 87.63) (width 0.4) (layer "B.Cu") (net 33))
 (segment (start 128.27 87.63) (end 133.35 87.63) (width 0.4) (layer "B.Cu") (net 33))
 (segment (start 133.35 87.63) (end 134.62 86.36) (width 0.4) (layer "B.Cu") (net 33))
 (segment (start 124.46 66.04) (end 125.611 64.889) (width 0.2) (layer "F.Cu") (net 50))
 (segment (start 125.611 64.889) (end 130.929 64.889) (width 0.2) (layer "F.Cu") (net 50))
 (segment (start 130.929 64.889) (end 132.08 66.04) (width 0.2) (layer "F.Cu") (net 50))
 (segment (start 127 127) (end 128.251 128.251) (width 0.4) (layer "B.Cu") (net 1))
 (segment (start 128.251 128.251) (end 133.369 128.251) (width 0.4) (layer "B.Cu") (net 1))
 (segment (start 133.369 128.251) (end 134.62 127) (width 0.4) (layer "B.Cu") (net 1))
 (segment (start 124.46 68.58) (end 125.611 67.429) (width 0.2) (layer "F.Cu") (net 48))
 (segment (start 130.929 67.429) (end 132.08 68.58) (width 0.2) (layer "F.Cu") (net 48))
 (segment (start 125.611 67.429) (end 130.929 67.429) (width 0.2) (layer "F.Cu") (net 48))
 (segment (start 125.611 97.909) (end 130.929 97.909) (width 0.2) (layer "F.Cu") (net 24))
 (segment (start 130.929 97.909) (end 132.08 99.06) (width 0.2) (layer "F.Cu") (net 24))
 (segment (start 124.46 99.06) (end 125.611 97.909) (width 0.2) (layer "F.Cu") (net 24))
 (segment (start 125.611 118.229) (end 130.929 118.229) (width 0.2) (layer "F.Cu") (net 8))
 (segment (start 124.46 119.38) (end 125.611 118.229) (width 0.2) (layer "F.Cu") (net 8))
 (segment (start 130.929 118.229) (end 132.08 119.38) (width 0.2) (layer "F.Cu") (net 8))
 (segment (start 131.3771 77.47) (end 133.35 77.47) (width 0.2) (layer "F.Cu") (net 41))
 (segment (start 130.1071 76.2) (end 131.3771 77.47) (width 0.2) (layer "F.Cu") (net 41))
 (segment (start 133.35 77.47) (end 134.62 76.2) (width 0.2) (layer "F.Cu") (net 41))
 (segment (start 127 76.2) (end 130.1071 76.2) (width 0.2) (layer "F.Cu") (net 41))
 (segment (start 130.1071 81.28) (end 131.3771 82.55) (width 0.2) (layer "F.Cu") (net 37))
 (segment (start 133.35 82.55) (end 134.62 81.28) (width 0.2) (layer "F.Cu") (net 37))
 (segment (start 127 81.28) (end 130.1071 81.28) (width 0.2) (layer "F.Cu") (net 37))
 (segment (start 131.3771 82.55) (end 133.35 82.55) (width 0.2) (layer "F.Cu") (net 37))
 (segment (start 125.849 92.591) (end 130.691 92.591) (width 0.2) (layer "F.Cu") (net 28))
 (segment (start 130.691 92.591) (end 132.08 93.98) (width 0.2) (layer "F.Cu") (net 28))
 (segment (start 124.46 93.98) (end 125.849 92.591) (width 0.2) (layer "F.Cu") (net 28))
 (segment (start 124.46 86.36) (end 125.611 85.209) (width 0.2) (layer "F.Cu") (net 34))
 (segment (start 125.611 85.209) (end 130.929 85.209) (width 0.2) (layer "F.Cu") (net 34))
 (segment (start 130.929 85.209) (end 132.08 86.36) (width 0.2) (layer "F.Cu") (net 34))
 (segment (start 130.691 120.531) (end 132.08 121.92) (width 0.2) (layer "F.Cu") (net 6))
 (segment (start 125.849 120.531) (end 130.691 120.531) (width 0.2) (layer "F.Cu") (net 6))
 (segment (start 124.46 121.92) (end 125.849 120.531) (width 0.2) (layer "F.Cu") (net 6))
 (segment (start 131.60324 100.211) (end 133.469 100.211) (width 0.2) (layer "F.Cu") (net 23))
 (segment (start 130.45224 99.06) (end 131.60324 100.211) (width 0.2) (layer "F.Cu") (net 23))
 (segment (start 133.469 100.211) (end 134.62 99.06) (width 0.2) (layer "F.Cu") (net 23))
 (segment (start 127 99.06) (end 130.45224 99.06) (width 0.2) (layer "F.Cu") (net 23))
 (segment (start 130.929 90.289) (end 132.08 91.44) (width 0.2) (layer "F.Cu") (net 30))
 (segment (start 124.46 91.44) (end 125.611 90.289) (width 0.2) (layer "F.Cu") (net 30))
 (segment (start 125.611 90.289) (end 130.929 90.289) (width 0.2) (layer "F.Cu") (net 30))
 (segment (start 130.1071 83.82) (end 131.3771 85.09) (width 0.2) (layer "F.Cu") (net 35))
 (segment (start 133.35 85.09) (end 134.62 83.82) (width 0.2) (layer "F.Cu") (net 35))
 (segment (start 131.3771 85.09) (end 133.35 85.09) (width 0.2) (layer "F.Cu") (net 35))
 (segment (start 127 83.82) (end 130.1071 83.82) (width 0.2) (layer "F.Cu") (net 35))
 (segment (start 131.60324 120.531) (end 133.469 120.531) (width 0.2) (layer "F.Cu") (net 7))
 (segment (start 127 119.38) (end 130.45224 119.38) (width 0.2) (layer "F.Cu") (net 7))
 (segment (start 130.45224 119.38) (end 131.60324 120.531) (width 0.2) (layer "F.Cu") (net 7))
 (segment (start 133.469 120.531) (end 134.62 119.38) (width 0.2) (layer "F.Cu") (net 7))
 (segment (start 130.21424 88.9) (end 131.36524 90.051) (width 0.2) (layer "F.Cu") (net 31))
 (segment (start 131.36524 90.051) (end 133.469 90.051) (width 0.2) (layer "F.Cu") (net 31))
 (segment (start 133.469 90.051) (end 134.62 88.9) (width 0.2) (layer "F.Cu") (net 31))
 (segment (start 127 88.9) (end 130.21424 88.9) (width 0.2) (layer "F.Cu") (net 31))
 (segment (start 130.45224 116.84) (end 131.60324 117.991) (width 0.2) (layer "F.Cu") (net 9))
 (segment (start 131.60324 117.991) (end 133.469 117.991) (width 0.2) (layer "F.Cu") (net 9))
 (segment (start 127 116.84) (end 130.45224 116.84) (width 0.2) (layer "F.Cu") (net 9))
 (segment (start 133.469 117.991) (end 134.62 116.84) (width 0.2) (layer "F.Cu") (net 9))
 (segment (start 131.60324 72.271) (end 133.469 72.271) (width 0.2) (layer "F.Cu") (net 45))
 (segment (start 127 71.12) (end 130.45224 71.12) (width 0.2) (layer "F.Cu") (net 45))
 (segment (start 133.469 72.271) (end 134.62 71.12) (width 0.2) (layer "F.Cu") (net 45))
 (segment (start 130.45224 71.12) (end 131.60324 72.271) (width 0.2) (layer "F.Cu") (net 45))
 (segment (start 133.469 79.891) (end 134.62 78.74) (width 0.2) (layer "F.Cu") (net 39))
 (segment (start 131.36524 79.891) (end 133.469 79.891) (width 0.2) (layer "F.Cu") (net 39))
 (segment (start 130.21424 78.74) (end 131.36524 79.891) (width 0.2) (layer "F.Cu") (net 39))
 (segment (start 127 78.74) (end 130.21424 78.74) (width 0.2) (layer "F.Cu") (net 39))
 (segment (start 125.611 110.609) (end 130.929 110.609) (width 0.2) (layer "F.Cu") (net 14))
 (segment (start 124.46 111.76) (end 125.611 110.609) (width 0.2) (layer "F.Cu") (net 14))
 (segment (start 130.929 110.609) (end 132.08 111.76) (width 0.2) (layer "F.Cu") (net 14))
 (segment (start 124.46 106.68) (end 125.611 105.529) (width 0.2) (layer "F.Cu") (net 18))
 (segment (start 125.611 105.529) (end 130.929 105.529) (width 0.2) (layer "F.Cu") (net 18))
 (segment (start 130.929 105.529) (end 132.08 106.68) (width 0.2) (layer "F.Cu") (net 18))
 (segment (start 125.611 72.509) (end 130.929 72.509) (width 0.2) (layer "F.Cu") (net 44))
 (segment (start 124.46 73.66) (end 125.611 72.509) (width 0.2) (layer "F.Cu") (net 44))
 (segment (start 130.929 72.509) (end 132.08 73.66) (width 0.2) (layer "F.Cu") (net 44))
 (segment (start 133.369 107.931) (end 134.62 106.68) (width 0.4) (layer "B.Cu") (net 17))
 (segment (start 128.251 107.931) (end 133.369 107.931) (width 0.4) (layer "B.Cu") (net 17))
 (segment (start 127 106.68) (end 128.251 107.931) (width 0.4) (layer "B.Cu") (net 17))
 (segment (start 130.929 75.049) (end 132.08 76.2) (width 0.2) (layer "F.Cu") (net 42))
 (segment (start 124.46 76.2) (end 125.611 75.049) (width 0.2) (layer "F.Cu") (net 42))
 (segment (start 125.611 75.049) (end 130.929 75.049) (width 0.2) (layer "F.Cu") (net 42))
 (segment (start 131.60324 112.911) (end 133.469 112.911) (width 0.2) (layer "F.Cu") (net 13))
 (segment (start 133.469 112.911) (end 134.62 111.76) (width 0.2) (layer "F.Cu") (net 13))
 (segment (start 127 111.76) (end 130.45224 111.76) (width 0.2) (layer "F.Cu") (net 13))
 (segment (start 130.45224 111.76) (end 131.60324 112.911) (width 0.2) (layer "F.Cu") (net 13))
 (segment (start 130.929 125.849) (end 132.08 127) (width 0.2) (layer "F.Cu") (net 2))
 (segment (start 125.611 125.849) (end 130.929 125.849) (width 0.2) (layer "F.Cu") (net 2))
 (segment (start 124.46 127) (end 125.611 125.849) (width 0.2) (layer "F.Cu") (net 2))
 (segment (start 130.45224 91.44) (end 131.60324 92.591) (width 0.2) (layer "F.Cu") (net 29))
 (segment (start 131.60324 92.591) (end 133.469 92.591) (width 0.2) (layer "F.Cu") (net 29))
 (segment (start 133.469 92.591) (end 134.62 91.44) (width 0.2) (layer "F.Cu") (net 29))
 (segment (start 127 91.44) (end 130.45224 91.44) (width 0.2) (layer "F.Cu") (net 29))
 (segment (start 127 109.22) (end 130.45224 109.22) (width 0.2) (layer "F.Cu") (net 15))
 (segment (start 130.45224 109.22) (end 131.60324 110.371) (width 0.2) (layer "F.Cu") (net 15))
 (segment (start 131.60324 110.371) (end 133.469 110.371) (width 0.2) (layer "F.Cu") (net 15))
 (segment (start 133.469 110.371) (end 134.62 109.22) (width 0.2) (layer "F.Cu") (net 15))
 (segment (start 125.611 113.149) (end 130.929 113.149) (width 0.2) (layer "F.Cu") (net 12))
 (segment (start 124.46 114.3) (end 125.611 113.149) (width 0.2) (layer "F.Cu") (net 12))
 (segment (start 130.929 113.149) (end 132.08 114.3) (width 0.2) (layer "F.Cu") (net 12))
 (segment (start 124.46 81.28) (end 125.611 80.129) (width 0.2) (layer "F.Cu") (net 38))
 (segment (start 130.929 80.129) (end 132.08 81.28) (width 0.2) (layer "F.Cu") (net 38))
 (segment (start 125.611 80.129) (end 130.929 80.129) (width 0.2) (layer "F.Cu") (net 38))
 (segment (start 125.73 95.25) (end 130.81 95.25) (width 0.2) (layer "F.Cu") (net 26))
 (segment (start 130.81 95.25) (end 132.08 96.52) (width 0.2) (layer "F.Cu") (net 26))
 (segment (start 124.46 96.52) (end 125.73 95.25) (width 0.2) (layer "F.Cu") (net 26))
 (segment (start 131.72224 69.85) (end 133.35 69.85) (width 0.2) (layer "F.Cu") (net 47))
 (segment (start 130.45224 68.58) (end 131.72224 69.85) (width 0.2) (layer "F.Cu") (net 47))
 (segment (start 127 68.58) (end 130.45224 68.58) (width 0.2) (layer "F.Cu") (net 47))
 (segment (start 133.35 69.85) (end 134.62 68.58) (width 0.2) (layer "F.Cu") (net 47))
 (segment (start 130.45224 104.14) (end 131.60324 105.291) (width 0.2) (layer "F.Cu") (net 19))
 (segment (start 133.469 105.291) (end 134.62 104.14) (width 0.2) (layer "F.Cu") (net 19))
 (segment (start 131.60324 105.291) (end 133.469 105.291) (width 0.2) (layer "F.Cu") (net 19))
 (segment (start 127 104.14) (end 130.45224 104.14) (width 0.2) (layer "F.Cu") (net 19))
 (segment (start 130.929 108.069) (end 132.08 109.22) (width 0.2) (layer "F.Cu") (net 16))
 (segment (start 124.46 109.22) (end 125.611 108.069) (width 0.2) (layer "F.Cu") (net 16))
 (segment (start 125.611 108.069) (end 130.929 108.069) (width 0.2) (layer "F.Cu") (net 16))
 (segment (start 127 93.98) (end 130.45224 93.98) (width 0.2) (layer "F.Cu") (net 27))
 (segment (start 131.60324 95.131) (end 133.469 95.131) (width 0.2) (layer "F.Cu") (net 27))
 (segment (start 133.469 95.131) (end 134.62 93.98) (width 0.2) (layer "F.Cu") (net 27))
 (segment (start 130.45224 93.98) (end 131.60324 95.131) (width 0.2) (layer "F.Cu") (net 27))
 (segment (start 124.46 78.74) (end 125.611 77.589) (width 0.2) (layer "F.Cu") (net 40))
 (segment (start 125.611 77.589) (end 130.929 77.589) (width 0.2) (layer "F.Cu") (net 40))
 (segment (start 130.929 77.589) (end 132.08 78.74) (width 0.2) (layer "F.Cu") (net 40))
 (segment (start 130.929 100.449) (end 132.08 101.6) (width 0.2) (layer "F.Cu") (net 22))
 (segment (start 125.611 100.449) (end 130.929 100.449) (width 0.2) (layer "F.Cu") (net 22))
 (segment (start 124.46 101.6) (end 125.611 100.449) (width 0.2) (layer "F.Cu") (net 22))
 (segment (start 133.369 67.291) (end 134.62 66.04) (width 0.4) (layer "B.Cu") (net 49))
 (segment (start 127 66.04) (end 128.251 67.291) (width 0.4) (layer "B.Cu") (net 49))
 (segment (start 128.251 67.291) (end 133.369 67.291) (width 0.4) (layer "B.Cu") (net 49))
 (segment (start 122.775 103.793) (end 122.775 134.078) (width 0.2) (layer "B.Cu") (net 21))
 (segment (start 134.62 134.112) (end 134.62 133.41) (width 0.2) (layer "B.Cu") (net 21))
 (segment (start 122.775 134.078) (end 123.444 134.747) (width 0.2) (layer "B.Cu") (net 21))
 (segment (start 123.444 134.747) (end 133.985 134.747) (width 0.2) (layer "B.Cu") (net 21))
 (segment (start 125.73 102.87) (end 123.698 102.87) (width 0.2) (layer "B.Cu") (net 21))
 (segment (start 133.985 134.747) (end 134.62 134.112) (width 0.2) (layer "B.Cu") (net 21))
 (segment (start 123.698 102.87) (end 122.775 103.793) (width 0.2) (layer "B.Cu") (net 21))
 (segment (start 127 101.6) (end 125.73 102.87) (width 0.2) (layer "B.Cu") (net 21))
 (segment (start 123.19 105.41) (end 124.46 104.14) (width 0.2) (layer "B.Cu") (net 20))
 (segment (start 124.714 133.35) (end 123.825 133.35) (width 0.2) (layer "B.Cu") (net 20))
 (segment (start 123.19 132.715) (end 123.19 105.41) (width 0.2) (layer "B.Cu") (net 20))
 (segment (start 123.825 133.35) (end 123.19 132.715) (width 0.2) (layer "B.Cu") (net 20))
 (segment (start 134.62 130.81) (end 136.051 129.379) (width 0.2) (layer "B.Cu") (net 54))
 (segment (start 136.051 103.031) (end 134.62 101.6) (width 0.2) (layer "B.Cu") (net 54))
 (segment (start 136.051 129.379) (end 136.051 103.031) (width 0.2) (layer "B.Cu") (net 54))
 (segment (start 124.714 130.75) (end 125.611 129.853) (width 0.2) (layer "B.Cu") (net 53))
 (segment (start 130.81 105.41) (end 132.08 104.14) (width 0.2) (layer "B.Cu") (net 53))
 (segment (start 125.611 106.291) (end 126.492 105.41) (width 0.2) (layer "B.Cu") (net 53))
 (segment (start 125.611 129.853) (end 125.611 106.291) (width 0.2) (layer "B.Cu") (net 53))
 (segment (start 126.492 105.41) (end 130.81 105.41) (width 0.2) (layer "B.Cu") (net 53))
 (segment (start 130.7 132.08) (end 134.59 132.08) (width 0.2) (layer "B.Cu") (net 51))
 (segment (start 134.59 132.08) (end 134.62 132.11) (width 0.2) (layer "B.Cu") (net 51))
 (segment (start 124.744 132.08) (end 124.714 132.05) (width 0.2) (layer "B.Cu") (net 52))
 (segment (start 128.16 132.08) (end 124.744 132.08) (width 0.2) (layer "B.Cu") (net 52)))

